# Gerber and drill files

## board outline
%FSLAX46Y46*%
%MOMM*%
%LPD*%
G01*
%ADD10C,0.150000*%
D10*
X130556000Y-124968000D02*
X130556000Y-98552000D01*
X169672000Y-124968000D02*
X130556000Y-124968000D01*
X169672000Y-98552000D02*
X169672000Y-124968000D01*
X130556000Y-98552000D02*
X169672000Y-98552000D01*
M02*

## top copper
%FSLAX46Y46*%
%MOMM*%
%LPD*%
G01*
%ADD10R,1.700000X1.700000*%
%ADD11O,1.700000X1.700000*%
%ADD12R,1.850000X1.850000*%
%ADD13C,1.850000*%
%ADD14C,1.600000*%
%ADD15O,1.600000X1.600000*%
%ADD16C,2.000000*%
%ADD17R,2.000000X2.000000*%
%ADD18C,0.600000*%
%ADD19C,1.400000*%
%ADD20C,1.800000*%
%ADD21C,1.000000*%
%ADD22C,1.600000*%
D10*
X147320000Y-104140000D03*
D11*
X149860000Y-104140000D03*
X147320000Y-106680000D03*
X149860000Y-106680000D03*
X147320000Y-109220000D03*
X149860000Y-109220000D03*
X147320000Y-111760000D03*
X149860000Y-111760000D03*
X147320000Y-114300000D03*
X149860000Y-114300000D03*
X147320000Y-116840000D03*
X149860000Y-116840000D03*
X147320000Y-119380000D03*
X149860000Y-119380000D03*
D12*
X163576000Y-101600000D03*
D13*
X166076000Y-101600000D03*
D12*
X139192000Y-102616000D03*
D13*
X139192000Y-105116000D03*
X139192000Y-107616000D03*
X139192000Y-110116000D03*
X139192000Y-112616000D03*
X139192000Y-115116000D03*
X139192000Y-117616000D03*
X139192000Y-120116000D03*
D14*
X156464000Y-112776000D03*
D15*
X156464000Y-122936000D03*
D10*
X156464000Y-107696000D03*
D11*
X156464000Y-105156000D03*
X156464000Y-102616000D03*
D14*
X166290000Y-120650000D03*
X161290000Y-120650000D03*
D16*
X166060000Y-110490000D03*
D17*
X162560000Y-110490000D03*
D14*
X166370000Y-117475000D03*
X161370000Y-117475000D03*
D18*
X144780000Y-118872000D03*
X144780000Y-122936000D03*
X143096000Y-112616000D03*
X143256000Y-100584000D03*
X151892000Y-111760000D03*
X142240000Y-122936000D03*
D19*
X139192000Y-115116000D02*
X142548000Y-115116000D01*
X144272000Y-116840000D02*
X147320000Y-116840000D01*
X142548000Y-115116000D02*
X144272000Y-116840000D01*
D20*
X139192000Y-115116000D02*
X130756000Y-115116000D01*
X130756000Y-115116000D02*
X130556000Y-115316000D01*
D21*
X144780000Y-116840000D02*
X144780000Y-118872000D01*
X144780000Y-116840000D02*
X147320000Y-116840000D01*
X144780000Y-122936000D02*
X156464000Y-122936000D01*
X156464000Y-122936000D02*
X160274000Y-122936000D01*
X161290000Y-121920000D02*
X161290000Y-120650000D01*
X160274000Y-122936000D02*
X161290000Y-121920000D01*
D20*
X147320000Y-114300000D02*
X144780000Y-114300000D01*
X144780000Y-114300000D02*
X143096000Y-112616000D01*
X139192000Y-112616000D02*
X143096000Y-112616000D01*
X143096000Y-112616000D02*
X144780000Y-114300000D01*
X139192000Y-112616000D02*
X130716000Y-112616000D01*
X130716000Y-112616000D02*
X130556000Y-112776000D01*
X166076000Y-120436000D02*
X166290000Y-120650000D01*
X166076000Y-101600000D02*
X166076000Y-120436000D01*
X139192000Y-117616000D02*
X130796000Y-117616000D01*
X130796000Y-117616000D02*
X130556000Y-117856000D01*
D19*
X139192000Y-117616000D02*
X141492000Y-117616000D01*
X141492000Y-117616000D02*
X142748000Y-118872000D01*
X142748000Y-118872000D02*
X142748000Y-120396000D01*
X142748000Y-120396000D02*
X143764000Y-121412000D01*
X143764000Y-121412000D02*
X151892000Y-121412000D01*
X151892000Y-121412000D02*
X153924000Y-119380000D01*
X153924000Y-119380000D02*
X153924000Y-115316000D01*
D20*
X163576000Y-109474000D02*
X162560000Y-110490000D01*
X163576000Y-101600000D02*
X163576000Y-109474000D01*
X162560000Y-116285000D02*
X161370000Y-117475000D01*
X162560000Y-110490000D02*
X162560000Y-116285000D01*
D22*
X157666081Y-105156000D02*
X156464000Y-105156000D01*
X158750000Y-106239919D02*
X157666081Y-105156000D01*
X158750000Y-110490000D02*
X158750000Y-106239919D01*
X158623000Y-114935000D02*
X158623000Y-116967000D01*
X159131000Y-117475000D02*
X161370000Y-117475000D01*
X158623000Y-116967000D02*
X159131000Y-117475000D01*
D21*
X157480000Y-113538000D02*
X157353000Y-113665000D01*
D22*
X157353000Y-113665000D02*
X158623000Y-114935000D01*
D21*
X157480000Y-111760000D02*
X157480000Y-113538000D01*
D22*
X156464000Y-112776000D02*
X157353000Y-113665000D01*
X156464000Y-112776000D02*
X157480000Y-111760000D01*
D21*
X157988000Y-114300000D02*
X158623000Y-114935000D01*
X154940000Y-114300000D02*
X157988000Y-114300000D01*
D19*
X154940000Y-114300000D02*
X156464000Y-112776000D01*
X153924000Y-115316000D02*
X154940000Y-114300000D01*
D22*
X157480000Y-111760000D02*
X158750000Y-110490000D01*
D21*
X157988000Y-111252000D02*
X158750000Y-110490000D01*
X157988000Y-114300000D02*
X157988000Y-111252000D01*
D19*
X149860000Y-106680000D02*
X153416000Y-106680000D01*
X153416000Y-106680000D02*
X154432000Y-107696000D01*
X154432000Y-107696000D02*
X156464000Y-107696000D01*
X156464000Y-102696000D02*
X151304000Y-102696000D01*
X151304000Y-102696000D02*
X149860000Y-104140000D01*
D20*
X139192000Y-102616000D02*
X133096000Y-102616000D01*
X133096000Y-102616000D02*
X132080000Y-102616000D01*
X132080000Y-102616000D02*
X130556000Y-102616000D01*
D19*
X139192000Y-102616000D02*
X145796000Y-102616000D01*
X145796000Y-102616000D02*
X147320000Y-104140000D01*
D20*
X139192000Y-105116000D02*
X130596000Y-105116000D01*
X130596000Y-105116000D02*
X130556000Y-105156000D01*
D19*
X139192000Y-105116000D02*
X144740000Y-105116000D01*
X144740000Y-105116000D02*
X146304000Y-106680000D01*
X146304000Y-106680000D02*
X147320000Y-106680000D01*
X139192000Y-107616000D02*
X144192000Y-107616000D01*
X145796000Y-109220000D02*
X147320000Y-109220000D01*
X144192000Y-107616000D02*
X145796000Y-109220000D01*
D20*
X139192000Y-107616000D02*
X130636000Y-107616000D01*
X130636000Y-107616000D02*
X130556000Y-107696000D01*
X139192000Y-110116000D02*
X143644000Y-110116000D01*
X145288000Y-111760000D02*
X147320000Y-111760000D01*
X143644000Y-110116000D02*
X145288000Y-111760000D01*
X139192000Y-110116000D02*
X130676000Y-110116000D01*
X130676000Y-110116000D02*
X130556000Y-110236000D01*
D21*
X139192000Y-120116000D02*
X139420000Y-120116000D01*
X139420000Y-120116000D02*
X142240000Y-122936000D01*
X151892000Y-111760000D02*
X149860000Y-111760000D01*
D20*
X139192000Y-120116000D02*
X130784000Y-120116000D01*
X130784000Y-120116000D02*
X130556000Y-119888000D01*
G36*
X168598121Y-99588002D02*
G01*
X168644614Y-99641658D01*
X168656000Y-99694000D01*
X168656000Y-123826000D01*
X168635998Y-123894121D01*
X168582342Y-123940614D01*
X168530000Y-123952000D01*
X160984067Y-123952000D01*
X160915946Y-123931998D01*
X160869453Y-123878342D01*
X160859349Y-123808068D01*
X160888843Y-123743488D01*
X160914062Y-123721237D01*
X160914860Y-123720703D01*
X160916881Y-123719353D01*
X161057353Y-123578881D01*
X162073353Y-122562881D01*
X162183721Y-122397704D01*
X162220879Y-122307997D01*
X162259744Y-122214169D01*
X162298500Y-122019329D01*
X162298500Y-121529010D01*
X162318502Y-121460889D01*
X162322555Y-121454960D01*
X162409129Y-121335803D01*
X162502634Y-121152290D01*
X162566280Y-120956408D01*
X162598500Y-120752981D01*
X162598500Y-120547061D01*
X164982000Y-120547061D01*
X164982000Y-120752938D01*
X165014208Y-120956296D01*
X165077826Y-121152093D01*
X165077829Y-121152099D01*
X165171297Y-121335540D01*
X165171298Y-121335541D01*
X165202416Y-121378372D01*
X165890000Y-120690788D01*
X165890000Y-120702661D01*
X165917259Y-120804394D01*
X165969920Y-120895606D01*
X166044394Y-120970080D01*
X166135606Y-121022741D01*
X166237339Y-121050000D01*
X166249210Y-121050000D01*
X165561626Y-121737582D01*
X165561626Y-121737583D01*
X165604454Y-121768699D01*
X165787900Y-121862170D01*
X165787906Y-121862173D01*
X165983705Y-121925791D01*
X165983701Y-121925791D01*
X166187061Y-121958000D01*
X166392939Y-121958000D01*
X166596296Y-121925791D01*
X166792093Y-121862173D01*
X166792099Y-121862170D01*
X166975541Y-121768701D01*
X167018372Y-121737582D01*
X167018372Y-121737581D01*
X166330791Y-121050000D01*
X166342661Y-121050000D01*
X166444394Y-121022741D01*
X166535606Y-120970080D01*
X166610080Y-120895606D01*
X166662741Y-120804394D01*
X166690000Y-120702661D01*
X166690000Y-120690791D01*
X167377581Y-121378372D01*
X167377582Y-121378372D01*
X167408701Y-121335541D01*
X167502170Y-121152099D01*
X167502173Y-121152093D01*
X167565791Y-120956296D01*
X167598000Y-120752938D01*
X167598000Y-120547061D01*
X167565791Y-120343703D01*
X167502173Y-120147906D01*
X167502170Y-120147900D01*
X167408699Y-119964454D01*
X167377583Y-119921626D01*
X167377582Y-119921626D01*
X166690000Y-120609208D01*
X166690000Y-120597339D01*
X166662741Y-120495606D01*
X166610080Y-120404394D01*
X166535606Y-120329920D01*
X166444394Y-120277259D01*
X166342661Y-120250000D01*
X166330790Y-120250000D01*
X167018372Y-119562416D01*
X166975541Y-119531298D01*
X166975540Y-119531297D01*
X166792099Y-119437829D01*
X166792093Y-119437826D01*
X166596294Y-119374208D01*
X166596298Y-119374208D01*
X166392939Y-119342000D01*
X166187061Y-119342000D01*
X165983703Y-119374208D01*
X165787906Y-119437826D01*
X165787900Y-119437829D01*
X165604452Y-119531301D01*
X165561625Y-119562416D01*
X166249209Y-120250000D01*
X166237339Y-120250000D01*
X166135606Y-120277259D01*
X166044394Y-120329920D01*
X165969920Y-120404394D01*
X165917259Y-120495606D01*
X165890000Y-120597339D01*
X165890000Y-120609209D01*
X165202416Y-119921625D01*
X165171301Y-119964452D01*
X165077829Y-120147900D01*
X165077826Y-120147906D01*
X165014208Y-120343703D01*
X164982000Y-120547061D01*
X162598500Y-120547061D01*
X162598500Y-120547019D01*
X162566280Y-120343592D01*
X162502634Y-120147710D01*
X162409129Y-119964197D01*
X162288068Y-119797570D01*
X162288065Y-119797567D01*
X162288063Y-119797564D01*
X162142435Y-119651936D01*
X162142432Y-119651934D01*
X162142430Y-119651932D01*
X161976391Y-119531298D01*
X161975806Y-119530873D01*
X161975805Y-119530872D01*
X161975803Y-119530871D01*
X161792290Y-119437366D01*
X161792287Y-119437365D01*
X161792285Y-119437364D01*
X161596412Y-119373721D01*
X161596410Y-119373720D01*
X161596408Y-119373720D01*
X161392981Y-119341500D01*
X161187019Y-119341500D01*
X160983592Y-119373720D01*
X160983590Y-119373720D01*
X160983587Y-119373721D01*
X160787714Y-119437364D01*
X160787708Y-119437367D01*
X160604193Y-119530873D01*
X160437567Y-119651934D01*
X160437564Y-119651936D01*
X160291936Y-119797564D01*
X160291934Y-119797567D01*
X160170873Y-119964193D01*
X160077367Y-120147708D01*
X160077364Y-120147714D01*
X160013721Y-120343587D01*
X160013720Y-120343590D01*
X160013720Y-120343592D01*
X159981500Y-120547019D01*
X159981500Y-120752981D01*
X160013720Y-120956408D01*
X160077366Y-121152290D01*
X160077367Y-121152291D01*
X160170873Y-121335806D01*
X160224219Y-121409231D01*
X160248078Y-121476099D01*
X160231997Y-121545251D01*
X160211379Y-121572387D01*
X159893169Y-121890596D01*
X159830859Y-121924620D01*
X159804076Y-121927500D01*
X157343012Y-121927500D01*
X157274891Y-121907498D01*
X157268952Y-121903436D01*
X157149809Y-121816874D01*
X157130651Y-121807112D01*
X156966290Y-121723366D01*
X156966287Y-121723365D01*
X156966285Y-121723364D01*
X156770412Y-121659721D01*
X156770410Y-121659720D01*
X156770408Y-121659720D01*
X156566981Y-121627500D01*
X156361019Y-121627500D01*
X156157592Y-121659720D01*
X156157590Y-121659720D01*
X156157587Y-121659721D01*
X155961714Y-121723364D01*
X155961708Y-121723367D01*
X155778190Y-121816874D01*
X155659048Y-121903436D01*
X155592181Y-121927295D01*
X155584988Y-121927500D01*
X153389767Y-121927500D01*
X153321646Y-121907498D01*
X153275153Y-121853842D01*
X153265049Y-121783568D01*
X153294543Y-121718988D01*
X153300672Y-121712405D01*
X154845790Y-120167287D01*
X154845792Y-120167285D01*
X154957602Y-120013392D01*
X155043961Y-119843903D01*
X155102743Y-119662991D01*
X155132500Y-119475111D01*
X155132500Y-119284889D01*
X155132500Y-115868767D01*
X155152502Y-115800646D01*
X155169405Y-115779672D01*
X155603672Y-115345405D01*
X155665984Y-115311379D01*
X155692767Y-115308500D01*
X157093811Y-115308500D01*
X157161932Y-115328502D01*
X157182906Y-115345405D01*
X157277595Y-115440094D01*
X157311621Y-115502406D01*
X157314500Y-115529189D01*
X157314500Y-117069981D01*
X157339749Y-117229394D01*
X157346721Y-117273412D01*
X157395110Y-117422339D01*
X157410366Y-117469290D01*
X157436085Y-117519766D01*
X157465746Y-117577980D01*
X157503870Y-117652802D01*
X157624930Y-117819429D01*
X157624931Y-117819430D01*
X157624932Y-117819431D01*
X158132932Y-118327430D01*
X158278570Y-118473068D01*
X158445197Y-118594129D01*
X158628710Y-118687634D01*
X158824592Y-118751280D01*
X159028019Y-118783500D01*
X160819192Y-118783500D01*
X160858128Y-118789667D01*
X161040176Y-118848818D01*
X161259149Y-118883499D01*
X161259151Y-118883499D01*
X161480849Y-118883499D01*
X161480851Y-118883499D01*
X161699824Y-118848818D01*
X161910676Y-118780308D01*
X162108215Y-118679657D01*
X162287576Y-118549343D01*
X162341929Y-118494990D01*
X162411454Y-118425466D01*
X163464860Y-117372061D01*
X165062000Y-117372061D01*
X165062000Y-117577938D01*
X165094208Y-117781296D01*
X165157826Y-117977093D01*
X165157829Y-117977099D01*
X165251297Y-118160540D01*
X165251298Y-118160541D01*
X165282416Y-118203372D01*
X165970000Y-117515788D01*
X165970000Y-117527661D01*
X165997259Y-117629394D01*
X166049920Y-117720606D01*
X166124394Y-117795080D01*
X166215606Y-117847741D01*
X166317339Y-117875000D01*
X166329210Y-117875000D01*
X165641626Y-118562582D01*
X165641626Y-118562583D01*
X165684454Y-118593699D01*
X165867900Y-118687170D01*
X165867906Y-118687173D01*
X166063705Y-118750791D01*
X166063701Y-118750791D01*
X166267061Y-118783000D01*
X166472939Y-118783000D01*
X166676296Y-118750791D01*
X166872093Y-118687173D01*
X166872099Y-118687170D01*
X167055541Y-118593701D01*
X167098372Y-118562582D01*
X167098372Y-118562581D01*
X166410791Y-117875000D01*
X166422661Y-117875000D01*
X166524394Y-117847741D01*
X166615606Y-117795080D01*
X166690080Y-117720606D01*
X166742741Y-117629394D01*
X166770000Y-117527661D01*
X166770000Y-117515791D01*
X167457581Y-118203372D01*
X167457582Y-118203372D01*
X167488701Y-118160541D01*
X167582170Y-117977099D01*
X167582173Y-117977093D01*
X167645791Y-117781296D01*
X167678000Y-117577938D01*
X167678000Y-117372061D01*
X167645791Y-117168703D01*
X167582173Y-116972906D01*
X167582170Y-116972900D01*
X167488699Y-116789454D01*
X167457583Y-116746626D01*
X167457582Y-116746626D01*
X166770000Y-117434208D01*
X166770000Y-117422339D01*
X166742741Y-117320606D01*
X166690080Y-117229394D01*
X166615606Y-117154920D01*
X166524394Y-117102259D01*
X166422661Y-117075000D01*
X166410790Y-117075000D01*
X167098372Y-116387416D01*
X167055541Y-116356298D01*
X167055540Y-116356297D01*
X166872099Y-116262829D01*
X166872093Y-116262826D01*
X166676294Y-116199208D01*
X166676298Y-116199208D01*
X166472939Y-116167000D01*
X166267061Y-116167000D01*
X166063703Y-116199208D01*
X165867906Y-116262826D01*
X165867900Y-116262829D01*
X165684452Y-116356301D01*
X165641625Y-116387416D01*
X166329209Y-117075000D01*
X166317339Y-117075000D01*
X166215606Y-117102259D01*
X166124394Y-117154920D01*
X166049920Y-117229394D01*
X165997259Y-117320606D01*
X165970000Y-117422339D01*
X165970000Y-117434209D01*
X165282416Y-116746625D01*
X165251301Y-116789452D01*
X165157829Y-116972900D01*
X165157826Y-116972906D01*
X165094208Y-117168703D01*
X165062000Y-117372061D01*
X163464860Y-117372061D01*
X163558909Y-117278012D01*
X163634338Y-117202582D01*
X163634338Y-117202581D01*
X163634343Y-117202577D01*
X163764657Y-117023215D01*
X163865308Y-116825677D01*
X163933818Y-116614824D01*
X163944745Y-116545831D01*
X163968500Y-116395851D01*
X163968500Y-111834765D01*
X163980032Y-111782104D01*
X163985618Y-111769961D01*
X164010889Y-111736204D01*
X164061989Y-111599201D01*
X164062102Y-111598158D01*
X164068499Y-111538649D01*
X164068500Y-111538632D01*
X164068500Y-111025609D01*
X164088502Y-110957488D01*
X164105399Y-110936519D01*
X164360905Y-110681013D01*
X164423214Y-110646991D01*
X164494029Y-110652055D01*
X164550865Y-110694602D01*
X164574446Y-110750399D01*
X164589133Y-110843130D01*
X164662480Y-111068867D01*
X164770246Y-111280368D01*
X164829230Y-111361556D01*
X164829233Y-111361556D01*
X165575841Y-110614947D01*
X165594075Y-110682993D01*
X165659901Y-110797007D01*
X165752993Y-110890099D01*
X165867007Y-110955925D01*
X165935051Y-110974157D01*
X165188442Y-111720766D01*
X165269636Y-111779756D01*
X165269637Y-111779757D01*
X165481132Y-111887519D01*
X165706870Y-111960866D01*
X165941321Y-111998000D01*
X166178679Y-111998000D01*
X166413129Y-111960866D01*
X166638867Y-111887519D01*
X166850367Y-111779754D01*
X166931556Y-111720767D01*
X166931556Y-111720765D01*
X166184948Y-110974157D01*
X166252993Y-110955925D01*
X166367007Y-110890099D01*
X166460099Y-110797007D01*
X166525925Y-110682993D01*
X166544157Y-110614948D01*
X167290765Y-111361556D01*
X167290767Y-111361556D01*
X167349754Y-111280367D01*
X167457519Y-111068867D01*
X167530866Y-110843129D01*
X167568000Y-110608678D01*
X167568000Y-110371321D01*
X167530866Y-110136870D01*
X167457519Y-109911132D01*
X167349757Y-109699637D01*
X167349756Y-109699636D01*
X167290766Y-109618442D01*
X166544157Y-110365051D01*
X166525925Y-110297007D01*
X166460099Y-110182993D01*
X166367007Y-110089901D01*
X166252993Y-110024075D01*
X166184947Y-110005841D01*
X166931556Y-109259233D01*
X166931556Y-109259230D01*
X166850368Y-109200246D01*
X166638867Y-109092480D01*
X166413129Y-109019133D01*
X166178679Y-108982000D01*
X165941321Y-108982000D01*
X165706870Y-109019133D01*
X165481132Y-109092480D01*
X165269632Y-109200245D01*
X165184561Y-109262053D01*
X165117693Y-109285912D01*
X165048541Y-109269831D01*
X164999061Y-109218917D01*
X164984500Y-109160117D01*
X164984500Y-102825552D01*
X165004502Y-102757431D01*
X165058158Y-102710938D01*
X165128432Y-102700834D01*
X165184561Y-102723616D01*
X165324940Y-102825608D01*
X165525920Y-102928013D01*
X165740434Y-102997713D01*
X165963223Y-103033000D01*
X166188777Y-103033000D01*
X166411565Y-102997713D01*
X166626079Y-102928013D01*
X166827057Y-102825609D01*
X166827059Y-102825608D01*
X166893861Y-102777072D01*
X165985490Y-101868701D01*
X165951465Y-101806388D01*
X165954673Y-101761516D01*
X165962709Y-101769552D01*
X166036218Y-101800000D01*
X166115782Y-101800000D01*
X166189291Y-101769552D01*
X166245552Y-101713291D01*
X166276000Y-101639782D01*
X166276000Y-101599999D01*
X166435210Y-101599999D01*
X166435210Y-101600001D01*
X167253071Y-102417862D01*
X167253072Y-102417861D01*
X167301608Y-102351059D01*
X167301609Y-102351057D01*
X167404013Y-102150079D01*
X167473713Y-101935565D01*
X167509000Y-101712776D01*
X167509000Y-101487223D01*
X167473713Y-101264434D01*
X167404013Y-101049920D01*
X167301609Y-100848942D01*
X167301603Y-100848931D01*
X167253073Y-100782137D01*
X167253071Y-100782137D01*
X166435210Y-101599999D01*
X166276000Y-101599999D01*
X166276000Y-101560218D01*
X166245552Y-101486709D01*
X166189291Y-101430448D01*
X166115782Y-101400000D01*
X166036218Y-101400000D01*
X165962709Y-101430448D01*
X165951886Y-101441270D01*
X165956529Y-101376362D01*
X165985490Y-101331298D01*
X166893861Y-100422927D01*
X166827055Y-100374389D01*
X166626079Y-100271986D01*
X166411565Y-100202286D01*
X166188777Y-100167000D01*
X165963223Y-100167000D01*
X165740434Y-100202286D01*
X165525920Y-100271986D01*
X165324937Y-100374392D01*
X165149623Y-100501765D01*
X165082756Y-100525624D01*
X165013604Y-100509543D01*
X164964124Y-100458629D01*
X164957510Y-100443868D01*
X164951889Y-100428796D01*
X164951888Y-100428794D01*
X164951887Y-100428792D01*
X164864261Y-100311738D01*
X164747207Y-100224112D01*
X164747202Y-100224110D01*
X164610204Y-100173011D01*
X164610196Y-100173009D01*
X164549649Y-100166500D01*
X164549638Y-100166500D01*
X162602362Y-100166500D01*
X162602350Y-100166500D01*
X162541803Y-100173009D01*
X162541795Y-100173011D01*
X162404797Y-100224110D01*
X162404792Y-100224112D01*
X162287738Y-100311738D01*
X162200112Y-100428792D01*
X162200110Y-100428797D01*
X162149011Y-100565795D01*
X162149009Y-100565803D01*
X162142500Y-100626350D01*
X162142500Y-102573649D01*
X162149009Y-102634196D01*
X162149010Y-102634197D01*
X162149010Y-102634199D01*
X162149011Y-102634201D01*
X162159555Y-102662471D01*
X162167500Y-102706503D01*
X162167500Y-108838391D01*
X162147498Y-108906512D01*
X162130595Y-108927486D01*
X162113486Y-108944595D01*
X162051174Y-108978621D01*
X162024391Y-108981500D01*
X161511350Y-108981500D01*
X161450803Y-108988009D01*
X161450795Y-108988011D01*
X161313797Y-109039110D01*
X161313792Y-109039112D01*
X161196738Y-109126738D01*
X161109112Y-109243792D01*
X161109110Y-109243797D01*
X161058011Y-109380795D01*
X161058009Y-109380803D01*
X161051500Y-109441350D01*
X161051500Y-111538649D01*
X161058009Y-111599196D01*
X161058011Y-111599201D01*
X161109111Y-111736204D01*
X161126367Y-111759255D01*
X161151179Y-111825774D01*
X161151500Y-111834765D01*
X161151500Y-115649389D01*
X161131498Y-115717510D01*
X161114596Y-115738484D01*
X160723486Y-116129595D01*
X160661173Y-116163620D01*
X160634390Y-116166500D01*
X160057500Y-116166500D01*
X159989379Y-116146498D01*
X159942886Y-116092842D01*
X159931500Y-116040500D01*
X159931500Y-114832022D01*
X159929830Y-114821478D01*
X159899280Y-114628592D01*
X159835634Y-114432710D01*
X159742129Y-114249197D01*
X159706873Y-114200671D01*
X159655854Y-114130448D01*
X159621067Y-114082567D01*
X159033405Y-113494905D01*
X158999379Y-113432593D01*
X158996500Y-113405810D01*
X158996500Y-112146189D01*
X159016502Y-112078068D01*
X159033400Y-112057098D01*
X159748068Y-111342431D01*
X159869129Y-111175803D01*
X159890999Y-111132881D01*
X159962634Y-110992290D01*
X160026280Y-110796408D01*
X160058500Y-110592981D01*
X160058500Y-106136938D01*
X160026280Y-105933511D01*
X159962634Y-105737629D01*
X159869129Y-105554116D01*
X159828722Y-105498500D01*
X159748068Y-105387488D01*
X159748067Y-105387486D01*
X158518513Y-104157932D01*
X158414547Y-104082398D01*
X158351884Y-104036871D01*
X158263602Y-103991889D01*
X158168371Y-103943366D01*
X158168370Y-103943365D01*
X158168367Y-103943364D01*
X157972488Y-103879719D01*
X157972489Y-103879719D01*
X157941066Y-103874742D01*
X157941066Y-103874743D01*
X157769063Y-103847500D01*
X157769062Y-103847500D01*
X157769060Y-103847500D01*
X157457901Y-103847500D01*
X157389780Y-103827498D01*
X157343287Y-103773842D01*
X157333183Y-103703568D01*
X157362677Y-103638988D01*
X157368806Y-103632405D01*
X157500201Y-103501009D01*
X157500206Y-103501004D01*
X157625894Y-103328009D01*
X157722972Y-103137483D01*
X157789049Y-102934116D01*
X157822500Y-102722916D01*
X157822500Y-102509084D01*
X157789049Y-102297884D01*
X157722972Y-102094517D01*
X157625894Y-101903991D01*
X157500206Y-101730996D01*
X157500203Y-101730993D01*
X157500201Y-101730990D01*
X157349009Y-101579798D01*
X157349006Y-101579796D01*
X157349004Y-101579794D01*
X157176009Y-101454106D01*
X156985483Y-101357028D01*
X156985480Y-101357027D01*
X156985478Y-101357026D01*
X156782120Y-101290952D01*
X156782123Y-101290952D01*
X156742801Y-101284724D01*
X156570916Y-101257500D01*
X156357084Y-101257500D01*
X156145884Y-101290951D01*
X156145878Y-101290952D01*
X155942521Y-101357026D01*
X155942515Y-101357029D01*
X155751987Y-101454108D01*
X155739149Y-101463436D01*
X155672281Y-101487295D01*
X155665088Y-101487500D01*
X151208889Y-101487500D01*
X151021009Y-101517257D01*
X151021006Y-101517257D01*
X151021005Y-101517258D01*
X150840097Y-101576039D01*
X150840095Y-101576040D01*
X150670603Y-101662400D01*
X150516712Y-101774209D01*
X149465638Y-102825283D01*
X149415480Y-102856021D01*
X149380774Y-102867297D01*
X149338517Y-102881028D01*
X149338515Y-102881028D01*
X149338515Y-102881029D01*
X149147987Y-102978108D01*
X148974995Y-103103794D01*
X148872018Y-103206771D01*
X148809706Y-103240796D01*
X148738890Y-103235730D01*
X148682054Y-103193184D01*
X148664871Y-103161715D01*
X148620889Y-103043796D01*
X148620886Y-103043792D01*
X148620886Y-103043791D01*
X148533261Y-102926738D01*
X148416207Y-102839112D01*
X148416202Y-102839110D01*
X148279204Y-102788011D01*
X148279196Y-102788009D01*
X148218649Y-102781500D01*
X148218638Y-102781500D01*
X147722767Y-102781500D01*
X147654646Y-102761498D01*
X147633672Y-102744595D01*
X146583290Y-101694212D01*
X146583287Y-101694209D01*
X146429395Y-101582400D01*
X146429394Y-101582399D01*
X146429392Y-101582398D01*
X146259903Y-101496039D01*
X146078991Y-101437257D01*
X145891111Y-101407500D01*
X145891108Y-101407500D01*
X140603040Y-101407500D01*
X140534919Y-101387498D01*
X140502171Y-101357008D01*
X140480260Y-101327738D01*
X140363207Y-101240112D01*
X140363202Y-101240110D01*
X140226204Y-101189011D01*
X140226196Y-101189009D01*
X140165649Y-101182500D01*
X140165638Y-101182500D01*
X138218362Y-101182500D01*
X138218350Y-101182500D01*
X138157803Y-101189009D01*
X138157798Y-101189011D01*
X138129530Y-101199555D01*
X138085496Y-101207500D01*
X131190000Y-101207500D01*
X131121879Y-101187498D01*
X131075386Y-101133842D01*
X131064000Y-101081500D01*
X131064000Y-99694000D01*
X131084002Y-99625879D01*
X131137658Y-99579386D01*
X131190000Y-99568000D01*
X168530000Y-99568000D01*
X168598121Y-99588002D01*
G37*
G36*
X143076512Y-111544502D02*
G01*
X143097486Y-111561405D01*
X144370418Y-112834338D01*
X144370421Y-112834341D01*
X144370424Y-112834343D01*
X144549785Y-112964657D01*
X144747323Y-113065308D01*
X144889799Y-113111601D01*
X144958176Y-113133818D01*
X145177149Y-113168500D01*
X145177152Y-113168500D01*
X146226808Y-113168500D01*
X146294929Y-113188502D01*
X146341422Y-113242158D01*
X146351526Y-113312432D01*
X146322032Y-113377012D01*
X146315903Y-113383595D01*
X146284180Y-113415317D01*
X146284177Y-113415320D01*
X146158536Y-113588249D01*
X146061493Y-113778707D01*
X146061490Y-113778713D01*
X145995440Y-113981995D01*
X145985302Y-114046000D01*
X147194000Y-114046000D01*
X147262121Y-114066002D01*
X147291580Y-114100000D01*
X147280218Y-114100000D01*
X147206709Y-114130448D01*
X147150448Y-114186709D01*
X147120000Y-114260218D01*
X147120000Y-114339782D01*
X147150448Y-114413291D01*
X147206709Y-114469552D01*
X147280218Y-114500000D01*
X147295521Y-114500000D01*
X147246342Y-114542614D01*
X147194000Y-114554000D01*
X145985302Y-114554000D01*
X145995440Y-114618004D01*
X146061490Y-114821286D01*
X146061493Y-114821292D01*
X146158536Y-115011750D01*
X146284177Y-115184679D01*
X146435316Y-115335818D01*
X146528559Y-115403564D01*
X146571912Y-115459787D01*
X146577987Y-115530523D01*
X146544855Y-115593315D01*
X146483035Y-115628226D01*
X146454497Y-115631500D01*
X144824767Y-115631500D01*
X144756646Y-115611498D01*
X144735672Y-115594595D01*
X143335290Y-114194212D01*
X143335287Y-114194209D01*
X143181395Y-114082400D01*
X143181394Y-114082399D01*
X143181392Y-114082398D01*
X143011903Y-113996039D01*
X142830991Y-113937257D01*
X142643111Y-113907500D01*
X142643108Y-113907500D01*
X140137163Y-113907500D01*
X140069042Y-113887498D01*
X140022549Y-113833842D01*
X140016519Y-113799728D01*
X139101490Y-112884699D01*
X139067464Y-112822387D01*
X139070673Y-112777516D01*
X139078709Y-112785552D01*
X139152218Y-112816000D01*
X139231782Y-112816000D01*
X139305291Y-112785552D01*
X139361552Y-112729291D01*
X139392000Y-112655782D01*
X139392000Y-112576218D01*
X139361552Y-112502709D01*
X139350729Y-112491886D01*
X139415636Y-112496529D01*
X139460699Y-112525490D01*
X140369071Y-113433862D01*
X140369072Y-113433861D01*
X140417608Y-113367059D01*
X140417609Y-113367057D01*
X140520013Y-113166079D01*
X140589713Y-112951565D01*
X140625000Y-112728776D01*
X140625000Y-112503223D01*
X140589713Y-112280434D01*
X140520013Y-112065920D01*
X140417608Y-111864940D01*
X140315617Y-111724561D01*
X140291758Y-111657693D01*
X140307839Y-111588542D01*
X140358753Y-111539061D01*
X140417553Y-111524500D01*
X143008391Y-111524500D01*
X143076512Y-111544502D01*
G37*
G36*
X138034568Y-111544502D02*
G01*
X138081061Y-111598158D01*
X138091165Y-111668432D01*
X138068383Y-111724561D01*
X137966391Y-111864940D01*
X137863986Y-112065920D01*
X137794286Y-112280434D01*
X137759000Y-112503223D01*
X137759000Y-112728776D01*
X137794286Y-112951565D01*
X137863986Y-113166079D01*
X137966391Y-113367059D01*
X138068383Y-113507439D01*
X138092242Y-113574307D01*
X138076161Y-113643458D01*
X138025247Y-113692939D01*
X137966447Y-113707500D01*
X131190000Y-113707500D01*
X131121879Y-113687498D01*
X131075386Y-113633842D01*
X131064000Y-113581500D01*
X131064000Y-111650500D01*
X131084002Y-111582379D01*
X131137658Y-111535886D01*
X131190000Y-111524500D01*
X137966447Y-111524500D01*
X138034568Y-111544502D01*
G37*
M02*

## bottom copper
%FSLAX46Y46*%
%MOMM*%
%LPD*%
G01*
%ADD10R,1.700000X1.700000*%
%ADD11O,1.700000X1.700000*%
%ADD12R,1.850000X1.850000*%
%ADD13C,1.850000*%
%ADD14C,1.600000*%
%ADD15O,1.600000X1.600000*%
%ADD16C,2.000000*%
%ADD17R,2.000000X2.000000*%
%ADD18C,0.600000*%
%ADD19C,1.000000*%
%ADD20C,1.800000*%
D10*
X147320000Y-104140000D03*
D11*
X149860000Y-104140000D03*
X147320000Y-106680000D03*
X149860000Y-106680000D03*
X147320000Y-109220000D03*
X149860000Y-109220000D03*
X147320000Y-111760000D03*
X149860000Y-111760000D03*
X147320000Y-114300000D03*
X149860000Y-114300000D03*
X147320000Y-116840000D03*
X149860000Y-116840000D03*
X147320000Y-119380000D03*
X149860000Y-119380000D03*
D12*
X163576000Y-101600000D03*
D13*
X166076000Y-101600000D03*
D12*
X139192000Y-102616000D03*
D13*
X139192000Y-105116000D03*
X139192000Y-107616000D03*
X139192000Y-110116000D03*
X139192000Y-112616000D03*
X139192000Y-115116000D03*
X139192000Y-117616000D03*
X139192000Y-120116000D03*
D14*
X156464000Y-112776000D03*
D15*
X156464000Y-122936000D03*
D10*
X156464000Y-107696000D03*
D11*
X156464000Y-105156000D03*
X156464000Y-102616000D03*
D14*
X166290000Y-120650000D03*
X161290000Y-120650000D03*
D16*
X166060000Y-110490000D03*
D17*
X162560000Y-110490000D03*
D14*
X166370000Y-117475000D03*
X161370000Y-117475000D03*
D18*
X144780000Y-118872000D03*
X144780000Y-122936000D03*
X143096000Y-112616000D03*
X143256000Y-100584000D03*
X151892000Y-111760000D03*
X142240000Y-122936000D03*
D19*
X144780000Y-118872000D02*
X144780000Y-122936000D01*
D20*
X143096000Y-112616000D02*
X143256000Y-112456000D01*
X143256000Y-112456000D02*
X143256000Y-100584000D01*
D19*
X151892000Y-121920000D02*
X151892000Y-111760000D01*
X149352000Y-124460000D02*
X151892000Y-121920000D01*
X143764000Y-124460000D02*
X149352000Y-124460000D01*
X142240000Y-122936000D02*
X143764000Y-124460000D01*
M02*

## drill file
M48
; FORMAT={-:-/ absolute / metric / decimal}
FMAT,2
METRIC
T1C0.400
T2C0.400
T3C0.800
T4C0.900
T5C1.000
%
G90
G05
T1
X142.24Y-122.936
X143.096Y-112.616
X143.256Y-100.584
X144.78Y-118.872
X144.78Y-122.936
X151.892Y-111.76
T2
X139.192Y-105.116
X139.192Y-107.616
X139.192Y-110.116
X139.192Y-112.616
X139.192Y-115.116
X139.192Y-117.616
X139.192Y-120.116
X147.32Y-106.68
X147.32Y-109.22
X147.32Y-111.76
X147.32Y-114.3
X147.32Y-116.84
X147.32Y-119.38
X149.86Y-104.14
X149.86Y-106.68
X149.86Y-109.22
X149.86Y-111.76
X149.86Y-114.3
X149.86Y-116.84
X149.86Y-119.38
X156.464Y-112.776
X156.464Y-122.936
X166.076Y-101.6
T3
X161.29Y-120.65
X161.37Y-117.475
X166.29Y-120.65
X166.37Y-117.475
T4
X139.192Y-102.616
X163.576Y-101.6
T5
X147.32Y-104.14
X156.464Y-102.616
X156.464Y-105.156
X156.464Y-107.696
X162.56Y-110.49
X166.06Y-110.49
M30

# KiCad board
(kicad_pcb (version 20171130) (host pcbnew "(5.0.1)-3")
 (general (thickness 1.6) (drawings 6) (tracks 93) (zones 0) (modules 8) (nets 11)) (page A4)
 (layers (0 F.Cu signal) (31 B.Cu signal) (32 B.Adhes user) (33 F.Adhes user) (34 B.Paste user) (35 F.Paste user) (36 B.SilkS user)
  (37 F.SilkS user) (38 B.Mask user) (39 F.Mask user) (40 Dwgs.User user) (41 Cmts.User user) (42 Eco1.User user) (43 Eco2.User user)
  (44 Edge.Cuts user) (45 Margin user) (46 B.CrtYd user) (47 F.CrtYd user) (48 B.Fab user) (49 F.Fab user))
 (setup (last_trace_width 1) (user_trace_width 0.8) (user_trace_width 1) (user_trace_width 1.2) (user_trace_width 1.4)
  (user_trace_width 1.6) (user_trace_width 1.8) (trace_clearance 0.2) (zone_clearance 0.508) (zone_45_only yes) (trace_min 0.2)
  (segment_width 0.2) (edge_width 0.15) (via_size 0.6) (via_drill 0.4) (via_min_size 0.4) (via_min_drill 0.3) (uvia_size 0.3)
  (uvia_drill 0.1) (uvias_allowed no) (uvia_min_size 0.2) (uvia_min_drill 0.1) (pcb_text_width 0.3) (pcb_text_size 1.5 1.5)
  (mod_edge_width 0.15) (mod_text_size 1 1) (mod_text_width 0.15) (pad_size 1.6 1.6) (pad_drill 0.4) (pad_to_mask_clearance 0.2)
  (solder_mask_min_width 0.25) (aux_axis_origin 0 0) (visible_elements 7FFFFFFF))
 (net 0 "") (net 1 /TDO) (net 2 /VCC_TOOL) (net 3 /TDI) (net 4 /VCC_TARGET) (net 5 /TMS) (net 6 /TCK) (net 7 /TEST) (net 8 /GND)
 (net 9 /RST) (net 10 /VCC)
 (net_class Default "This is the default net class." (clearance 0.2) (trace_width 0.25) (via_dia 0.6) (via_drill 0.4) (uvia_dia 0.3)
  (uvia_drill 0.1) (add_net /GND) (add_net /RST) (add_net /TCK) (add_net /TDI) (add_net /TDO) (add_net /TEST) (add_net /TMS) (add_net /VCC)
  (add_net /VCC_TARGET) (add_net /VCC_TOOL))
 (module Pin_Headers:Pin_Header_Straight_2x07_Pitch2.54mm (layer F.Cu) (at 147.32 104.14)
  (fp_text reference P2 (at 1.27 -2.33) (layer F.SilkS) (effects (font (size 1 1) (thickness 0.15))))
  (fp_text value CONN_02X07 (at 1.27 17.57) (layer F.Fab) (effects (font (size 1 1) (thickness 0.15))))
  (pad 1 thru_hole rect (at 0 0) (size 1.7 1.7) (drill 1) (layers *.Cu *.Mask) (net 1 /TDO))
  (pad 2 thru_hole oval (at 2.54 0) (size 1.7 1.7) (drill 0.4) (layers *.Cu *.Mask) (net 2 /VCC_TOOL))
  (pad 3 thru_hole oval (at 0 2.54) (size 1.7 1.7) (drill 0.4) (layers *.Cu *.Mask) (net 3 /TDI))
  (pad 4 thru_hole oval (at 2.54 2.54) (size 1.7 1.7) (drill 0.4) (layers *.Cu *.Mask) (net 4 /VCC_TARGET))
  (pad 5 thru_hole oval (at 0 5.08) (size 1.7 1.7) (drill 0.4) (layers *.Cu *.Mask) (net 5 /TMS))
  (pad 6 thru_hole oval (at 2.54 5.08) (size 1.7 1.7) (drill 0.4) (layers *.Cu *.Mask))
  (pad 7 thru_hole oval (at 0 7.62) (size 1.7 1.7) (drill 0.4) (layers *.Cu *.Mask) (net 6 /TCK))
  (pad 8 thru_hole oval (at 2.54 7.62) (size 1.7 1.7) (drill 0.4) (layers *.Cu *.Mask) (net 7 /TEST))
  (pad 9 thru_hole oval (at 0 10.16) (size 1.7 1.7) (drill 0.4) (layers *.Cu *.Mask) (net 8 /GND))
  (pad 10 thru_hole oval (at 2.54 10.16) (size 1.7 1.7) (drill 0.4) (layers *.Cu *.Mask))
  (pad 11 thru_hole oval (at 0 12.7) (size 1.7 1.7) (drill 0.4) (layers *.Cu *.Mask) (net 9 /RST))
  (pad 12 thru_hole oval (at 2.54 12.7) (size 1.7 1.7) (drill 0.4) (layers *.Cu *.Mask))
  (pad 13 thru_hole oval (at 0 15.24) (size 1.7 1.7) (drill 0.4) (layers *.Cu *.Mask))
  (pad 14 thru_hole oval (at 2.54 15.24) (size 1.7 1.7) (drill 0.4) (layers *.Cu *.Mask)))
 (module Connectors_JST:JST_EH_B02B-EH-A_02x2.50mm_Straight (layer F.Cu) (at 163.576 101.6)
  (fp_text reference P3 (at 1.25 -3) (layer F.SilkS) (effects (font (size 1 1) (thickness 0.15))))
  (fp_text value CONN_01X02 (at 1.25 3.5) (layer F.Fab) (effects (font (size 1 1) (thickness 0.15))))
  (pad 1 thru_hole rect (at 0 0) (size 1.85 1.85) (drill 0.9) (layers *.Cu *.Mask) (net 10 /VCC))
  (pad 2 thru_hole circle (at 2.5 0) (size 1.85 1.85) (drill 0.4) (layers *.Cu *.Mask) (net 8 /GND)))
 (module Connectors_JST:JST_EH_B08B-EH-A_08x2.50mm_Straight (layer F.Cu) (at 139.192 102.616 270)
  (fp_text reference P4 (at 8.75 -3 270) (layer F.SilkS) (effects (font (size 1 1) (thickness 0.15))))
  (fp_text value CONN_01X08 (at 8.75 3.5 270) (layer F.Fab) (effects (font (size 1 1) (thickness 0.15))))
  (pad 1 thru_hole rect (at 0 0 270) (size 1.85 1.85) (drill 0.9) (layers *.Cu *.Mask) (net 1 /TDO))
  (pad 2 thru_hole circle (at 2.5 0 270) (size 1.85 1.85) (drill 0.4) (layers *.Cu *.Mask) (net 3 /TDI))
  (pad 3 thru_hole circle (at 5 0 270) (size 1.85 1.85) (drill 0.4) (layers *.Cu *.Mask) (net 5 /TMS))
  (pad 4 thru_hole circle (at 7.5 0 270) (size 1.85 1.85) (drill 0.4) (layers *.Cu *.Mask) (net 6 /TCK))
  (pad 5 thru_hole circle (at 10 0 270) (size 1.85 1.85) (drill 0.4) (layers *.Cu *.Mask) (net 8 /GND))
  (pad 6 thru_hole circle (at 12.5 0 270) (size 1.85 1.85) (drill 0.4) (layers *.Cu *.Mask) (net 9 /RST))
  (pad 7 thru_hole circle (at 15 0 270) (size 1.85 1.85) (drill 0.4) (layers *.Cu *.Mask) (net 10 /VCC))
  (pad 8 thru_hole circle (at 17.5 0 270) (size 1.85 1.85) (drill 0.4) (layers *.Cu *.Mask) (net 7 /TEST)))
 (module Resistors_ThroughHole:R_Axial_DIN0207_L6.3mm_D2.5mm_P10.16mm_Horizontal (layer F.Cu) (at 156.464 112.776 270)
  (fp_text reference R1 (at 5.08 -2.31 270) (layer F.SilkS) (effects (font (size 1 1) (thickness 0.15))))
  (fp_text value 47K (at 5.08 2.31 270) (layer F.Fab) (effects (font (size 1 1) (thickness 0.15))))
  (pad 1 thru_hole circle (at 0 0 270) (size 1.6 1.6) (drill 0.4) (layers *.Cu *.Mask) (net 10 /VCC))
  (pad 2 thru_hole oval (at 10.16 0 270) (size 1.6 1.6) (drill 0.4) (layers *.Cu *.Mask) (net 9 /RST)))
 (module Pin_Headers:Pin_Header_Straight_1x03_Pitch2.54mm (layer F.Cu) (at 156.464 107.696 180)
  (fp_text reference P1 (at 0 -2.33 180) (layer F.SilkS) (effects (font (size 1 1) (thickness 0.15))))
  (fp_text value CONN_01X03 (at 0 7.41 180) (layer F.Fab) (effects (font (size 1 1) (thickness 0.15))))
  (pad 1 thru_hole rect (at 0 0 180) (size 1.7 1.7) (drill 1) (layers *.Cu *.Mask) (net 4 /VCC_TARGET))
  (pad 2 thru_hole oval (at 0 2.54 180) (size 1.7 1.7) (drill 1) (layers *.Cu *.Mask) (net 10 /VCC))
  (pad 3 thru_hole oval (at 0 5.08 180) (size 1.7 1.7) (drill 1) (layers *.Cu *.Mask) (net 2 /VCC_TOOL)))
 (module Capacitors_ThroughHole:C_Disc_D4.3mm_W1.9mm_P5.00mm (layer F.Cu) (at 161.29 120.65)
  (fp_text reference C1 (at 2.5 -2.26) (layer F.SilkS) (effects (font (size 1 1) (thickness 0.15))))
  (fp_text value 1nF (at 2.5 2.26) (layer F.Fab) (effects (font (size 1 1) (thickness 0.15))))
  (pad 2 thru_hole circle (at 5 0) (size 1.6 1.6) (drill 0.8) (layers *.Cu *.Mask) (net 8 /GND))
  (pad 1 thru_hole circle (at 0 0) (size 1.6 1.6) (drill 0.8) (layers *.Cu *.Mask) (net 9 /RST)))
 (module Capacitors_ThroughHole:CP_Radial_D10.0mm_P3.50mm (layer F.Cu) (at 162.56 110.49)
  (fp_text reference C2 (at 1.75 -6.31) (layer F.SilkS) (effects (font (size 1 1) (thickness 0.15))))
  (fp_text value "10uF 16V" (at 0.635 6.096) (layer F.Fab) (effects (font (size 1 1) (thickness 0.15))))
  (pad 2 thru_hole circle (at 3.5 0) (size 2 2) (drill 1) (layers *.Cu *.Mask) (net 8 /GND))
  (pad 1 thru_hole rect (at 0 0) (size 2 2) (drill 1) (layers *.Cu *.Mask) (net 10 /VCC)))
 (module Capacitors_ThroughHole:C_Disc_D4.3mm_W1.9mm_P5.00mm (layer F.Cu) (at 166.37 117.475 180)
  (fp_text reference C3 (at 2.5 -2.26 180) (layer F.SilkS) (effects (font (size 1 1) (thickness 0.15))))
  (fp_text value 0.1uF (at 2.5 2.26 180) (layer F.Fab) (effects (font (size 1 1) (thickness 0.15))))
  (pad 1 thru_hole circle (at 0 0 180) (size 1.6 1.6) (drill 0.8) (layers *.Cu *.Mask) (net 8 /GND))
  (pad 2 thru_hole circle (at 5 0 180) (size 1.6 1.6) (drill 0.8) (layers *.Cu *.Mask) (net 10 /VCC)))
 (gr_line (start 130.556 124.968) (end 130.556 98.552) (angle 90) (layer Edge.Cuts) (width 0.15))
 (gr_line (start 169.672 124.968) (end 130.556 124.968) (angle 90) (layer Edge.Cuts) (width 0.15))
 (gr_line (start 169.672 98.552) (end 169.672 124.968) (angle 90) (layer Edge.Cuts) (width 0.15))
 (gr_line (start 130.556 98.552) (end 169.672 98.552) (angle 90) (layer Edge.Cuts) (width 0.15))
 (segment (start 139.192 115.116) (end 142.548 115.116) (width 1.4) (layer F.Cu) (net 9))
 (segment (start 144.272 116.84) (end 147.32 116.84) (width 1.4) (layer F.Cu) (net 9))
 (segment (start 142.548 115.116) (end 144.272 116.84) (width 1.4) (layer F.Cu) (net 9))
 (segment (start 139.192 115.116) (end 130.756 115.116) (width 1.8) (layer F.Cu) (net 9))
 (segment (start 130.756 115.116) (end 130.556 115.316) (width 1.8) (layer F.Cu) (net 9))
 (segment (start 144.78 116.84) (end 144.78 118.872) (width 1) (layer F.Cu) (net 9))
 (segment (start 144.78 116.84) (end 147.32 116.84) (width 1) (layer F.Cu) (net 9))
 (via (at 144.78 118.872) (size 0.6) (drill 0.4) (layers F.Cu B.Cu) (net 9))
 (segment (start 144.78 118.872) (end 144.78 122.936) (width 1) (layer B.Cu) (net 9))
 (via (at 144.78 122.936) (size 0.6) (drill 0.4) (layers F.Cu B.Cu) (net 9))
 (segment (start 144.78 122.936) (end 156.464 122.936) (width 1) (layer F.Cu) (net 9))
 (segment (start 156.464 122.936) (end 160.274 122.936) (width 1) (layer F.Cu) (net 9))
 (segment (start 161.29 121.92) (end 161.29 120.65) (width 1) (layer F.Cu) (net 9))
 (segment (start 160.274 122.936) (end 161.29 121.92) (width 1) (layer F.Cu) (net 9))
 (segment (start 147.32 114.3) (end 144.78 114.3) (width 1.8) (layer F.Cu) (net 8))
 (segment (start 144.78 114.3) (end 143.096 112.616) (width 1.8) (layer F.Cu) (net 8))
 (via (at 143.096 112.616) (size 0.6) (drill 0.4) (layers F.Cu B.Cu) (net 8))
 (segment (start 143.096 112.616) (end 143.256 112.456) (width 1.8) (layer B.Cu) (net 8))
 (segment (start 143.256 112.456) (end 143.256 100.584) (width 1.8) (layer B.Cu) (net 8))
 (via (at 143.256 100.584) (size 0.6) (drill 0.4) (layers F.Cu B.Cu) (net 8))
 (segment (start 139.192 112.616) (end 143.096 112.616) (width 1.8) (layer F.Cu) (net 8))
 (segment (start 143.096 112.616) (end 144.78 114.3) (width 1.8) (layer F.Cu) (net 8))
 (segment (start 139.192 112.616) (end 130.716 112.616) (width 1.8) (layer F.Cu) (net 8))
 (segment (start 130.716 112.616) (end 130.556 112.776) (width 1.8) (layer F.Cu) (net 8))
 (segment (start 166.076 120.436) (end 166.29 120.65) (width 1.8) (layer F.Cu) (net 8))
 (segment (start 166.076 101.6) (end 166.076 120.436) (width 1.8) (layer F.Cu) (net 8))
 (segment (start 139.192 117.616) (end 130.796 117.616) (width 1.8) (layer F.Cu) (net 10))
 (segment (start 130.796 117.616) (end 130.556 117.856) (width 1.8) (layer F.Cu) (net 10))
 (segment (start 139.192 117.616) (end 141.492 117.616) (width 1.4) (layer F.Cu) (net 10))
 (segment (start 141.492 117.616) (end 142.748 118.872) (width 1.4) (layer F.Cu) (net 10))
 (segment (start 142.748 118.872) (end 142.748 120.396) (width 1.4) (layer F.Cu) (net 10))
 (segment (start 142.748 120.396) (end 143.764 121.412) (width 1.4) (layer F.Cu) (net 10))
 (segment (start 143.764 121.412) (end 151.892 121.412) (width 1.4) (layer F.Cu) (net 10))
 (segment (start 151.892 121.412) (end 153.924 119.38) (width 1.4) (layer F.Cu) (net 10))
 (segment (start 153.924 119.38) (end 153.924 115.316) (width 1.4) (layer F.Cu) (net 10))
 (segment (start 163.576 109.474) (end 162.56 110.49) (width 1.8) (layer F.Cu) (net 10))
 (segment (start 163.576 101.6) (end 163.576 109.474) (width 1.8) (layer F.Cu) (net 10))
 (segment (start 162.56 116.285) (end 161.37 117.475) (width 1.8) (layer F.Cu) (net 10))
 (segment (start 162.56 110.49) (end 162.56 116.285) (width 1.8) (layer F.Cu) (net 10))
 (segment (start 157.666081 105.156) (end 156.464 105.156) (width 1.6) (layer F.Cu) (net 10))
 (segment (start 158.75 106.239919) (end 157.666081 105.156) (width 1.6) (layer F.Cu) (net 10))
 (segment (start 158.75 110.49) (end 158.75 106.239919) (width 1.6) (layer F.Cu) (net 10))
 (segment (start 158.623 114.935) (end 158.623 116.967) (width 1.6) (layer F.Cu) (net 10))
 (segment (start 159.131 117.475) (end 161.37 117.475) (width 1.6) (layer F.Cu) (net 10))
 (segment (start 158.623 116.967) (end 159.131 117.475) (width 1.6) (layer F.Cu) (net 10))
 (segment (start 157.48 113.538) (end 157.353 113.665) (width 1) (layer F.Cu) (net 10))
 (segment (start 157.353 113.665) (end 158.623 114.935) (width 1.6) (layer F.Cu) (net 10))
 (segment (start 157.48 111.76) (end 157.48 113.538) (width 1) (layer F.Cu) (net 10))
 (segment (start 156.464 112.776) (end 157.353 113.665) (width 1.6) (layer F.Cu) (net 10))
 (segment (start 156.464 112.776) (end 157.48 111.76) (width 1.6) (layer F.Cu) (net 10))
 (segment (start 157.988 114.3) (end 158.623 114.935) (width 1) (layer F.Cu) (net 10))
 (segment (start 154.94 114.3) (end 157.988 114.3) (width 1) (layer F.Cu) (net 10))
 (segment (start 154.94 114.3) (end 156.464 112.776) (width 1.4) (layer F.Cu) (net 10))
 (segment (start 153.924 115.316) (end 154.94 114.3) (width 1.4) (layer F.Cu) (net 10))
 (segment (start 157.48 111.76) (end 158.75 110.49) (width 1.6) (layer F.Cu) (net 10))
 (segment (start 157.988 111.252) (end 158.75 110.49) (width 1) (layer F.Cu) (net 10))
 (segment (start 157.988 114.3) (end 157.988 111.252) (width 1) (layer F.Cu) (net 10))
 (segment (start 149.86 106.68) (end 153.416 106.68) (width 1.4) (layer F.Cu) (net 4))
 (segment (start 153.416 106.68) (end 154.432 107.696) (width 1.4) (layer F.Cu) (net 4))
 (segment (start 154.432 107.696) (end 156.464 107.696) (width 1.4) (layer F.Cu) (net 4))
 (segment (start 156.464 102.696) (end 151.304 102.696) (width 1.4) (layer F.Cu) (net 2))
 (segment (start 151.304 102.696) (end 149.86 104.14) (width 1.4) (layer F.Cu) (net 2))
 (segment (start 139.192 102.616) (end 133.096 102.616) (width 1.8) (layer F.Cu) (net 1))
 (segment (start 133.096 102.616) (end 132.08 102.616) (width 1.8) (layer F.Cu) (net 1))
 (segment (start 132.08 102.616) (end 130.556 102.616) (width 1.8) (layer F.Cu) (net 1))
 (segment (start 139.192 102.616) (end 145.796 102.616) (width 1.4) (layer F.Cu) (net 1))
 (segment (start 145.796 102.616) (end 147.32 104.14) (width 1.4) (layer F.Cu) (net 1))
 (segment (start 139.192 105.116) (end 130.596 105.116) (width 1.8) (layer F.Cu) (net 3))
 (segment (start 130.596 105.116) (end 130.556 105.156) (width 1.8) (layer F.Cu) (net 3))
 (segment (start 139.192 105.116) (end 144.74 105.116) (width 1.4) (layer F.Cu) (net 3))
 (segment (start 144.74 105.116) (end 146.304 106.68) (width 1.4) (layer F.Cu) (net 3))
 (segment (start 146.304 106.68) (end 147.32 106.68) (width 1.4) (layer F.Cu) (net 3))
 (segment (start 139.192 107.616) (end 144.192 107.616) (width 1.4) (layer F.Cu) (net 5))
 (segment (start 145.796 109.22) (end 147.32 109.22) (width 1.4) (layer F.Cu) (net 5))
 (segment (start 144.192 107.616) (end 145.796 109.22) (width 1.4) (layer F.Cu) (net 5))
 (segment (start 139.192 107.616) (end 130.636 107.616) (width 1.8) (layer F.Cu) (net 5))
 (segment (start 130.636 107.616) (end 130.556 107.696) (width 1.8) (layer F.Cu) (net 5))
 (segment (start 139.192 110.116) (end 143.644 110.116) (width 1.8) (layer F.Cu) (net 6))
 (segment (start 145.288 111.76) (end 147.32 111.76) (width 1.8) (layer F.Cu) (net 6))
 (segment (start 143.644 110.116) (end 145.288 111.76) (width 1.8) (layer F.Cu) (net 6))
 (segment (start 139.192 110.116) (end 130.676 110.116) (width 1.8) (layer F.Cu) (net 6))
 (segment (start 130.676 110.116) (end 130.556 110.236) (width 1.8) (layer F.Cu) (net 6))
 (segment (start 139.192 120.116) (end 139.42 120.116) (width 1) (layer F.Cu) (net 7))
 (segment (start 139.42 120.116) (end 142.24 122.936) (width 1) (layer F.Cu) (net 7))
 (segment (start 151.892 111.76) (end 149.86 111.76) (width 1) (layer F.Cu) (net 7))
 (via (at 151.892 111.76) (size 0.6) (drill 0.4) (layers F.Cu B.Cu) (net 7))
 (segment (start 151.892 121.92) (end 151.892 111.76) (width 1) (layer B.Cu) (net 7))
 (segment (start 149.352 124.46) (end 151.892 121.92) (width 1) (layer B.Cu) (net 7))
 (segment (start 143.764 124.46) (end 149.352 124.46) (width 1) (layer B.Cu) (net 7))
 (segment (start 142.24 122.936) (end 143.764 124.46) (width 1) (layer B.Cu) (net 7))
 (via (at 142.24 122.936) (size 0.6) (drill 0.4) (layers F.Cu B.Cu) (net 7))
 (segment (start 139.192 120.116) (end 130.784 120.116) (width 1.8) (layer F.Cu) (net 7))
 (segment (start 130.784 120.116) (end 130.556 119.888) (width 1.8) (layer F.Cu) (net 7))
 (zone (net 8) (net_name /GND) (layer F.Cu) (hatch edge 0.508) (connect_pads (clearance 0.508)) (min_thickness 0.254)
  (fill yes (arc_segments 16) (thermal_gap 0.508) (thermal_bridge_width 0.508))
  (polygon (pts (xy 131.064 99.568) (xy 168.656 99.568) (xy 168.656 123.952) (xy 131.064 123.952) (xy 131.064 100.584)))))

